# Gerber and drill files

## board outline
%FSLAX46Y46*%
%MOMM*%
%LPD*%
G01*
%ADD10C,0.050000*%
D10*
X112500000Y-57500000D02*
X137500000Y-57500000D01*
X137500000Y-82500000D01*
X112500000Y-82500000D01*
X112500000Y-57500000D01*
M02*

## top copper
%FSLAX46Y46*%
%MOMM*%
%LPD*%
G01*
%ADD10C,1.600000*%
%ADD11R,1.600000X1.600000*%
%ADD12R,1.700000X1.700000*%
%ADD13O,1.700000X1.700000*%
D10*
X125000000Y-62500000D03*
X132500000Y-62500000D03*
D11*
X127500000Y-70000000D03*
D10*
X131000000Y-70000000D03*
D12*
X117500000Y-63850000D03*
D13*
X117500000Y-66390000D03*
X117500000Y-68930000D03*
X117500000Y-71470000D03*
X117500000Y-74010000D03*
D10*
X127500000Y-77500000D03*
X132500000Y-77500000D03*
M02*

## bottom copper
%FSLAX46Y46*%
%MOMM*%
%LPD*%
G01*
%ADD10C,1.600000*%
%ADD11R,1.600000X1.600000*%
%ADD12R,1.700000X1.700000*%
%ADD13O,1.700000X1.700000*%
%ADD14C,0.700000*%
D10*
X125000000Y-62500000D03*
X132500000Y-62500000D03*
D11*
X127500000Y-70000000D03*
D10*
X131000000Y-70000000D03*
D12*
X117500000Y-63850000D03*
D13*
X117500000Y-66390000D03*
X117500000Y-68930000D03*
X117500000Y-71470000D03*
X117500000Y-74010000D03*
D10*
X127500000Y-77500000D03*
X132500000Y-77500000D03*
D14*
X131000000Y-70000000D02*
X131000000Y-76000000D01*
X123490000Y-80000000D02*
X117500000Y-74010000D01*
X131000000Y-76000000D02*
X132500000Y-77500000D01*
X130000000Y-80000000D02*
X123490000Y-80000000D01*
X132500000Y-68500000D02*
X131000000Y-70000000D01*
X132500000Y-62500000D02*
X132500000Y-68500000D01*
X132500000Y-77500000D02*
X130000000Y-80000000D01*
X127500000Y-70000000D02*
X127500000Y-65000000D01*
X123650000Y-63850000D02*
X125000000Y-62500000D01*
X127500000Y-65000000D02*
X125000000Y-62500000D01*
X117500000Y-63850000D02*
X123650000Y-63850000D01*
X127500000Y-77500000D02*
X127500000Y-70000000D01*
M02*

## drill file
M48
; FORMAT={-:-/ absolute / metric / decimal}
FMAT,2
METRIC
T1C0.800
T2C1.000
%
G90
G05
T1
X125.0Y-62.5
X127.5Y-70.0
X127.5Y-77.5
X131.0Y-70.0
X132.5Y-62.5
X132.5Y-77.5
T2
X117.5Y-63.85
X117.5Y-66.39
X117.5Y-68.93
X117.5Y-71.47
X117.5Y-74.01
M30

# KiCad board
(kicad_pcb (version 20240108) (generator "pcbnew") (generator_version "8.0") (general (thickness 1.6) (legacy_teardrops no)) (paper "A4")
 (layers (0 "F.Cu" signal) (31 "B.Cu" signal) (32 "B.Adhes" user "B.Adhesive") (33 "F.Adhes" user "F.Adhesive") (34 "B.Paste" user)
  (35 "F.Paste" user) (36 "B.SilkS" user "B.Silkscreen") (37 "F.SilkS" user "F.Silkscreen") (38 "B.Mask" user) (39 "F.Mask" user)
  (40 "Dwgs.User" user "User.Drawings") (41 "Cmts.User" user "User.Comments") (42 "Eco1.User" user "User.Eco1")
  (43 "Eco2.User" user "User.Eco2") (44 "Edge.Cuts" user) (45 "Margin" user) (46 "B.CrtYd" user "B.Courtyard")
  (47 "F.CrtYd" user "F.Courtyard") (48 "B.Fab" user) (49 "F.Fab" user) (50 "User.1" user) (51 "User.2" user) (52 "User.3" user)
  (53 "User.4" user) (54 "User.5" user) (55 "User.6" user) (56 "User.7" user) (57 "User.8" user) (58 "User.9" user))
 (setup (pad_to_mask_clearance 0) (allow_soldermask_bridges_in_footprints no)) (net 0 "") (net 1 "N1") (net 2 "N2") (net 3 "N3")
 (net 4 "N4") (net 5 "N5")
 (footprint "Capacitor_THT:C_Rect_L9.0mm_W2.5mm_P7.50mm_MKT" (layer "F.Cu") (at 125 62.5)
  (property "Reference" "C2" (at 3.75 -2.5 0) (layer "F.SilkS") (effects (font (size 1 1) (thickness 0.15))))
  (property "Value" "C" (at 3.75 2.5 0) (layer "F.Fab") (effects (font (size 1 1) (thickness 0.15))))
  (pad "1" thru_hole circle (at 0 0) (size 1.6 1.6) (drill 0.8) (layers "*.Cu" "*.Mask") (remove_unused_layers no) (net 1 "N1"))
  (pad "2" thru_hole circle (at 7.5 0) (size 1.6 1.6) (drill 0.8) (layers "*.Cu" "*.Mask") (remove_unused_layers no) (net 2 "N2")))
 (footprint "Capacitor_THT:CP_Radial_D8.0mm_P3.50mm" (layer "F.Cu") (at 127.5 70)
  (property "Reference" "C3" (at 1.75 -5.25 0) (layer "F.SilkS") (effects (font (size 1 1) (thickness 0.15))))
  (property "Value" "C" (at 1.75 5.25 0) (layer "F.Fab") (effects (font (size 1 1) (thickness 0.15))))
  (pad "1" thru_hole rect (at 0 0) (size 1.6 1.6) (drill 0.8) (layers "*.Cu" "*.Mask") (remove_unused_layers no) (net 1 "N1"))
  (pad "2" thru_hole circle (at 3.5 0) (size 1.6 1.6) (drill 0.8) (layers "*.Cu" "*.Mask") (remove_unused_layers no) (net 2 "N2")))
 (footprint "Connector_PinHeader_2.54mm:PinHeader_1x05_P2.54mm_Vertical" (layer "F.Cu") (at 117.5 63.85)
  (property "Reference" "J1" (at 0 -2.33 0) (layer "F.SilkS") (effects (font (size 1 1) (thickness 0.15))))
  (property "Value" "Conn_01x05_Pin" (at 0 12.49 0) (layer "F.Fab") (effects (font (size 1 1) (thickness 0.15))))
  (pad "1" thru_hole rect (at 0 0) (size 1.7 1.7) (drill 1) (layers "*.Cu" "*.Mask") (remove_unused_layers no) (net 1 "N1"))
  (pad "2" thru_hole oval (at 0 2.54) (size 1.7 1.7) (drill 1) (layers "*.Cu" "*.Mask") (remove_unused_layers no) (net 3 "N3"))
  (pad "3" thru_hole oval (at 0 5.08) (size 1.7 1.7) (drill 1) (layers "*.Cu" "*.Mask") (remove_unused_layers no) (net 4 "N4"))
  (pad "4" thru_hole oval (at 0 7.62) (size 1.7 1.7) (drill 1) (layers "*.Cu" "*.Mask") (remove_unused_layers no) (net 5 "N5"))
  (pad "5" thru_hole oval (at 0 10.16) (size 1.7 1.7) (drill 1) (layers "*.Cu" "*.Mask") (remove_unused_layers no) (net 2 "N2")))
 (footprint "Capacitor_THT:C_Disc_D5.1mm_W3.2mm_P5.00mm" (layer "F.Cu") (at 127.5 77.5)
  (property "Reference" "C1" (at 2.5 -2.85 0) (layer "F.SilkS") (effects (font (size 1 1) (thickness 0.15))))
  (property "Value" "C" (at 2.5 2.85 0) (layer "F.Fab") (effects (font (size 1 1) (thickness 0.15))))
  (pad "1" thru_hole circle (at 0 0) (size 1.6 1.6) (drill 0.8) (layers "*.Cu" "*.Mask") (remove_unused_layers no) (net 1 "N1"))
  (pad "2" thru_hole circle (at 5 0) (size 1.6 1.6) (drill 0.8) (layers "*.Cu" "*.Mask") (remove_unused_layers no) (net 2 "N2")))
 (gr_rect (start 112.5 57.5) (end 137.5 82.5) (stroke (width 0.05) (type default)) (fill none) (layer "Edge.Cuts"))
 (segment (start 131 70) (end 131 76) (width 0.7) (layer "B.Cu") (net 2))
 (segment (start 123.49 80) (end 117.5 74.01) (width 0.7) (layer "B.Cu") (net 2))
 (segment (start 131 76) (end 132.5 77.5) (width 0.7) (layer "B.Cu") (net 2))
 (segment (start 130 80) (end 123.49 80) (width 0.7) (layer "B.Cu") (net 2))
 (segment (start 132.5 68.5) (end 131 70) (width 0.7) (layer "B.Cu") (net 2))
 (segment (start 132.5 62.5) (end 132.5 68.5) (width 0.7) (layer "B.Cu") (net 2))
 (segment (start 132.5 77.5) (end 130 80) (width 0.7) (layer "B.Cu") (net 2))
 (segment (start 127.5 70) (end 127.5 65) (width 0.7) (layer "B.Cu") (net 1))
 (segment (start 123.65 63.85) (end 125 62.5) (width 0.7) (layer "B.Cu") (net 1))
 (segment (start 127.5 65) (end 125 62.5) (width 0.7) (layer "B.Cu") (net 1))
 (segment (start 117.5 63.85) (end 123.65 63.85) (width 0.7) (layer "B.Cu") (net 1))
 (segment (start 127.5 77.5) (end 127.5 70) (width 0.7) (layer "B.Cu") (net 1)))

